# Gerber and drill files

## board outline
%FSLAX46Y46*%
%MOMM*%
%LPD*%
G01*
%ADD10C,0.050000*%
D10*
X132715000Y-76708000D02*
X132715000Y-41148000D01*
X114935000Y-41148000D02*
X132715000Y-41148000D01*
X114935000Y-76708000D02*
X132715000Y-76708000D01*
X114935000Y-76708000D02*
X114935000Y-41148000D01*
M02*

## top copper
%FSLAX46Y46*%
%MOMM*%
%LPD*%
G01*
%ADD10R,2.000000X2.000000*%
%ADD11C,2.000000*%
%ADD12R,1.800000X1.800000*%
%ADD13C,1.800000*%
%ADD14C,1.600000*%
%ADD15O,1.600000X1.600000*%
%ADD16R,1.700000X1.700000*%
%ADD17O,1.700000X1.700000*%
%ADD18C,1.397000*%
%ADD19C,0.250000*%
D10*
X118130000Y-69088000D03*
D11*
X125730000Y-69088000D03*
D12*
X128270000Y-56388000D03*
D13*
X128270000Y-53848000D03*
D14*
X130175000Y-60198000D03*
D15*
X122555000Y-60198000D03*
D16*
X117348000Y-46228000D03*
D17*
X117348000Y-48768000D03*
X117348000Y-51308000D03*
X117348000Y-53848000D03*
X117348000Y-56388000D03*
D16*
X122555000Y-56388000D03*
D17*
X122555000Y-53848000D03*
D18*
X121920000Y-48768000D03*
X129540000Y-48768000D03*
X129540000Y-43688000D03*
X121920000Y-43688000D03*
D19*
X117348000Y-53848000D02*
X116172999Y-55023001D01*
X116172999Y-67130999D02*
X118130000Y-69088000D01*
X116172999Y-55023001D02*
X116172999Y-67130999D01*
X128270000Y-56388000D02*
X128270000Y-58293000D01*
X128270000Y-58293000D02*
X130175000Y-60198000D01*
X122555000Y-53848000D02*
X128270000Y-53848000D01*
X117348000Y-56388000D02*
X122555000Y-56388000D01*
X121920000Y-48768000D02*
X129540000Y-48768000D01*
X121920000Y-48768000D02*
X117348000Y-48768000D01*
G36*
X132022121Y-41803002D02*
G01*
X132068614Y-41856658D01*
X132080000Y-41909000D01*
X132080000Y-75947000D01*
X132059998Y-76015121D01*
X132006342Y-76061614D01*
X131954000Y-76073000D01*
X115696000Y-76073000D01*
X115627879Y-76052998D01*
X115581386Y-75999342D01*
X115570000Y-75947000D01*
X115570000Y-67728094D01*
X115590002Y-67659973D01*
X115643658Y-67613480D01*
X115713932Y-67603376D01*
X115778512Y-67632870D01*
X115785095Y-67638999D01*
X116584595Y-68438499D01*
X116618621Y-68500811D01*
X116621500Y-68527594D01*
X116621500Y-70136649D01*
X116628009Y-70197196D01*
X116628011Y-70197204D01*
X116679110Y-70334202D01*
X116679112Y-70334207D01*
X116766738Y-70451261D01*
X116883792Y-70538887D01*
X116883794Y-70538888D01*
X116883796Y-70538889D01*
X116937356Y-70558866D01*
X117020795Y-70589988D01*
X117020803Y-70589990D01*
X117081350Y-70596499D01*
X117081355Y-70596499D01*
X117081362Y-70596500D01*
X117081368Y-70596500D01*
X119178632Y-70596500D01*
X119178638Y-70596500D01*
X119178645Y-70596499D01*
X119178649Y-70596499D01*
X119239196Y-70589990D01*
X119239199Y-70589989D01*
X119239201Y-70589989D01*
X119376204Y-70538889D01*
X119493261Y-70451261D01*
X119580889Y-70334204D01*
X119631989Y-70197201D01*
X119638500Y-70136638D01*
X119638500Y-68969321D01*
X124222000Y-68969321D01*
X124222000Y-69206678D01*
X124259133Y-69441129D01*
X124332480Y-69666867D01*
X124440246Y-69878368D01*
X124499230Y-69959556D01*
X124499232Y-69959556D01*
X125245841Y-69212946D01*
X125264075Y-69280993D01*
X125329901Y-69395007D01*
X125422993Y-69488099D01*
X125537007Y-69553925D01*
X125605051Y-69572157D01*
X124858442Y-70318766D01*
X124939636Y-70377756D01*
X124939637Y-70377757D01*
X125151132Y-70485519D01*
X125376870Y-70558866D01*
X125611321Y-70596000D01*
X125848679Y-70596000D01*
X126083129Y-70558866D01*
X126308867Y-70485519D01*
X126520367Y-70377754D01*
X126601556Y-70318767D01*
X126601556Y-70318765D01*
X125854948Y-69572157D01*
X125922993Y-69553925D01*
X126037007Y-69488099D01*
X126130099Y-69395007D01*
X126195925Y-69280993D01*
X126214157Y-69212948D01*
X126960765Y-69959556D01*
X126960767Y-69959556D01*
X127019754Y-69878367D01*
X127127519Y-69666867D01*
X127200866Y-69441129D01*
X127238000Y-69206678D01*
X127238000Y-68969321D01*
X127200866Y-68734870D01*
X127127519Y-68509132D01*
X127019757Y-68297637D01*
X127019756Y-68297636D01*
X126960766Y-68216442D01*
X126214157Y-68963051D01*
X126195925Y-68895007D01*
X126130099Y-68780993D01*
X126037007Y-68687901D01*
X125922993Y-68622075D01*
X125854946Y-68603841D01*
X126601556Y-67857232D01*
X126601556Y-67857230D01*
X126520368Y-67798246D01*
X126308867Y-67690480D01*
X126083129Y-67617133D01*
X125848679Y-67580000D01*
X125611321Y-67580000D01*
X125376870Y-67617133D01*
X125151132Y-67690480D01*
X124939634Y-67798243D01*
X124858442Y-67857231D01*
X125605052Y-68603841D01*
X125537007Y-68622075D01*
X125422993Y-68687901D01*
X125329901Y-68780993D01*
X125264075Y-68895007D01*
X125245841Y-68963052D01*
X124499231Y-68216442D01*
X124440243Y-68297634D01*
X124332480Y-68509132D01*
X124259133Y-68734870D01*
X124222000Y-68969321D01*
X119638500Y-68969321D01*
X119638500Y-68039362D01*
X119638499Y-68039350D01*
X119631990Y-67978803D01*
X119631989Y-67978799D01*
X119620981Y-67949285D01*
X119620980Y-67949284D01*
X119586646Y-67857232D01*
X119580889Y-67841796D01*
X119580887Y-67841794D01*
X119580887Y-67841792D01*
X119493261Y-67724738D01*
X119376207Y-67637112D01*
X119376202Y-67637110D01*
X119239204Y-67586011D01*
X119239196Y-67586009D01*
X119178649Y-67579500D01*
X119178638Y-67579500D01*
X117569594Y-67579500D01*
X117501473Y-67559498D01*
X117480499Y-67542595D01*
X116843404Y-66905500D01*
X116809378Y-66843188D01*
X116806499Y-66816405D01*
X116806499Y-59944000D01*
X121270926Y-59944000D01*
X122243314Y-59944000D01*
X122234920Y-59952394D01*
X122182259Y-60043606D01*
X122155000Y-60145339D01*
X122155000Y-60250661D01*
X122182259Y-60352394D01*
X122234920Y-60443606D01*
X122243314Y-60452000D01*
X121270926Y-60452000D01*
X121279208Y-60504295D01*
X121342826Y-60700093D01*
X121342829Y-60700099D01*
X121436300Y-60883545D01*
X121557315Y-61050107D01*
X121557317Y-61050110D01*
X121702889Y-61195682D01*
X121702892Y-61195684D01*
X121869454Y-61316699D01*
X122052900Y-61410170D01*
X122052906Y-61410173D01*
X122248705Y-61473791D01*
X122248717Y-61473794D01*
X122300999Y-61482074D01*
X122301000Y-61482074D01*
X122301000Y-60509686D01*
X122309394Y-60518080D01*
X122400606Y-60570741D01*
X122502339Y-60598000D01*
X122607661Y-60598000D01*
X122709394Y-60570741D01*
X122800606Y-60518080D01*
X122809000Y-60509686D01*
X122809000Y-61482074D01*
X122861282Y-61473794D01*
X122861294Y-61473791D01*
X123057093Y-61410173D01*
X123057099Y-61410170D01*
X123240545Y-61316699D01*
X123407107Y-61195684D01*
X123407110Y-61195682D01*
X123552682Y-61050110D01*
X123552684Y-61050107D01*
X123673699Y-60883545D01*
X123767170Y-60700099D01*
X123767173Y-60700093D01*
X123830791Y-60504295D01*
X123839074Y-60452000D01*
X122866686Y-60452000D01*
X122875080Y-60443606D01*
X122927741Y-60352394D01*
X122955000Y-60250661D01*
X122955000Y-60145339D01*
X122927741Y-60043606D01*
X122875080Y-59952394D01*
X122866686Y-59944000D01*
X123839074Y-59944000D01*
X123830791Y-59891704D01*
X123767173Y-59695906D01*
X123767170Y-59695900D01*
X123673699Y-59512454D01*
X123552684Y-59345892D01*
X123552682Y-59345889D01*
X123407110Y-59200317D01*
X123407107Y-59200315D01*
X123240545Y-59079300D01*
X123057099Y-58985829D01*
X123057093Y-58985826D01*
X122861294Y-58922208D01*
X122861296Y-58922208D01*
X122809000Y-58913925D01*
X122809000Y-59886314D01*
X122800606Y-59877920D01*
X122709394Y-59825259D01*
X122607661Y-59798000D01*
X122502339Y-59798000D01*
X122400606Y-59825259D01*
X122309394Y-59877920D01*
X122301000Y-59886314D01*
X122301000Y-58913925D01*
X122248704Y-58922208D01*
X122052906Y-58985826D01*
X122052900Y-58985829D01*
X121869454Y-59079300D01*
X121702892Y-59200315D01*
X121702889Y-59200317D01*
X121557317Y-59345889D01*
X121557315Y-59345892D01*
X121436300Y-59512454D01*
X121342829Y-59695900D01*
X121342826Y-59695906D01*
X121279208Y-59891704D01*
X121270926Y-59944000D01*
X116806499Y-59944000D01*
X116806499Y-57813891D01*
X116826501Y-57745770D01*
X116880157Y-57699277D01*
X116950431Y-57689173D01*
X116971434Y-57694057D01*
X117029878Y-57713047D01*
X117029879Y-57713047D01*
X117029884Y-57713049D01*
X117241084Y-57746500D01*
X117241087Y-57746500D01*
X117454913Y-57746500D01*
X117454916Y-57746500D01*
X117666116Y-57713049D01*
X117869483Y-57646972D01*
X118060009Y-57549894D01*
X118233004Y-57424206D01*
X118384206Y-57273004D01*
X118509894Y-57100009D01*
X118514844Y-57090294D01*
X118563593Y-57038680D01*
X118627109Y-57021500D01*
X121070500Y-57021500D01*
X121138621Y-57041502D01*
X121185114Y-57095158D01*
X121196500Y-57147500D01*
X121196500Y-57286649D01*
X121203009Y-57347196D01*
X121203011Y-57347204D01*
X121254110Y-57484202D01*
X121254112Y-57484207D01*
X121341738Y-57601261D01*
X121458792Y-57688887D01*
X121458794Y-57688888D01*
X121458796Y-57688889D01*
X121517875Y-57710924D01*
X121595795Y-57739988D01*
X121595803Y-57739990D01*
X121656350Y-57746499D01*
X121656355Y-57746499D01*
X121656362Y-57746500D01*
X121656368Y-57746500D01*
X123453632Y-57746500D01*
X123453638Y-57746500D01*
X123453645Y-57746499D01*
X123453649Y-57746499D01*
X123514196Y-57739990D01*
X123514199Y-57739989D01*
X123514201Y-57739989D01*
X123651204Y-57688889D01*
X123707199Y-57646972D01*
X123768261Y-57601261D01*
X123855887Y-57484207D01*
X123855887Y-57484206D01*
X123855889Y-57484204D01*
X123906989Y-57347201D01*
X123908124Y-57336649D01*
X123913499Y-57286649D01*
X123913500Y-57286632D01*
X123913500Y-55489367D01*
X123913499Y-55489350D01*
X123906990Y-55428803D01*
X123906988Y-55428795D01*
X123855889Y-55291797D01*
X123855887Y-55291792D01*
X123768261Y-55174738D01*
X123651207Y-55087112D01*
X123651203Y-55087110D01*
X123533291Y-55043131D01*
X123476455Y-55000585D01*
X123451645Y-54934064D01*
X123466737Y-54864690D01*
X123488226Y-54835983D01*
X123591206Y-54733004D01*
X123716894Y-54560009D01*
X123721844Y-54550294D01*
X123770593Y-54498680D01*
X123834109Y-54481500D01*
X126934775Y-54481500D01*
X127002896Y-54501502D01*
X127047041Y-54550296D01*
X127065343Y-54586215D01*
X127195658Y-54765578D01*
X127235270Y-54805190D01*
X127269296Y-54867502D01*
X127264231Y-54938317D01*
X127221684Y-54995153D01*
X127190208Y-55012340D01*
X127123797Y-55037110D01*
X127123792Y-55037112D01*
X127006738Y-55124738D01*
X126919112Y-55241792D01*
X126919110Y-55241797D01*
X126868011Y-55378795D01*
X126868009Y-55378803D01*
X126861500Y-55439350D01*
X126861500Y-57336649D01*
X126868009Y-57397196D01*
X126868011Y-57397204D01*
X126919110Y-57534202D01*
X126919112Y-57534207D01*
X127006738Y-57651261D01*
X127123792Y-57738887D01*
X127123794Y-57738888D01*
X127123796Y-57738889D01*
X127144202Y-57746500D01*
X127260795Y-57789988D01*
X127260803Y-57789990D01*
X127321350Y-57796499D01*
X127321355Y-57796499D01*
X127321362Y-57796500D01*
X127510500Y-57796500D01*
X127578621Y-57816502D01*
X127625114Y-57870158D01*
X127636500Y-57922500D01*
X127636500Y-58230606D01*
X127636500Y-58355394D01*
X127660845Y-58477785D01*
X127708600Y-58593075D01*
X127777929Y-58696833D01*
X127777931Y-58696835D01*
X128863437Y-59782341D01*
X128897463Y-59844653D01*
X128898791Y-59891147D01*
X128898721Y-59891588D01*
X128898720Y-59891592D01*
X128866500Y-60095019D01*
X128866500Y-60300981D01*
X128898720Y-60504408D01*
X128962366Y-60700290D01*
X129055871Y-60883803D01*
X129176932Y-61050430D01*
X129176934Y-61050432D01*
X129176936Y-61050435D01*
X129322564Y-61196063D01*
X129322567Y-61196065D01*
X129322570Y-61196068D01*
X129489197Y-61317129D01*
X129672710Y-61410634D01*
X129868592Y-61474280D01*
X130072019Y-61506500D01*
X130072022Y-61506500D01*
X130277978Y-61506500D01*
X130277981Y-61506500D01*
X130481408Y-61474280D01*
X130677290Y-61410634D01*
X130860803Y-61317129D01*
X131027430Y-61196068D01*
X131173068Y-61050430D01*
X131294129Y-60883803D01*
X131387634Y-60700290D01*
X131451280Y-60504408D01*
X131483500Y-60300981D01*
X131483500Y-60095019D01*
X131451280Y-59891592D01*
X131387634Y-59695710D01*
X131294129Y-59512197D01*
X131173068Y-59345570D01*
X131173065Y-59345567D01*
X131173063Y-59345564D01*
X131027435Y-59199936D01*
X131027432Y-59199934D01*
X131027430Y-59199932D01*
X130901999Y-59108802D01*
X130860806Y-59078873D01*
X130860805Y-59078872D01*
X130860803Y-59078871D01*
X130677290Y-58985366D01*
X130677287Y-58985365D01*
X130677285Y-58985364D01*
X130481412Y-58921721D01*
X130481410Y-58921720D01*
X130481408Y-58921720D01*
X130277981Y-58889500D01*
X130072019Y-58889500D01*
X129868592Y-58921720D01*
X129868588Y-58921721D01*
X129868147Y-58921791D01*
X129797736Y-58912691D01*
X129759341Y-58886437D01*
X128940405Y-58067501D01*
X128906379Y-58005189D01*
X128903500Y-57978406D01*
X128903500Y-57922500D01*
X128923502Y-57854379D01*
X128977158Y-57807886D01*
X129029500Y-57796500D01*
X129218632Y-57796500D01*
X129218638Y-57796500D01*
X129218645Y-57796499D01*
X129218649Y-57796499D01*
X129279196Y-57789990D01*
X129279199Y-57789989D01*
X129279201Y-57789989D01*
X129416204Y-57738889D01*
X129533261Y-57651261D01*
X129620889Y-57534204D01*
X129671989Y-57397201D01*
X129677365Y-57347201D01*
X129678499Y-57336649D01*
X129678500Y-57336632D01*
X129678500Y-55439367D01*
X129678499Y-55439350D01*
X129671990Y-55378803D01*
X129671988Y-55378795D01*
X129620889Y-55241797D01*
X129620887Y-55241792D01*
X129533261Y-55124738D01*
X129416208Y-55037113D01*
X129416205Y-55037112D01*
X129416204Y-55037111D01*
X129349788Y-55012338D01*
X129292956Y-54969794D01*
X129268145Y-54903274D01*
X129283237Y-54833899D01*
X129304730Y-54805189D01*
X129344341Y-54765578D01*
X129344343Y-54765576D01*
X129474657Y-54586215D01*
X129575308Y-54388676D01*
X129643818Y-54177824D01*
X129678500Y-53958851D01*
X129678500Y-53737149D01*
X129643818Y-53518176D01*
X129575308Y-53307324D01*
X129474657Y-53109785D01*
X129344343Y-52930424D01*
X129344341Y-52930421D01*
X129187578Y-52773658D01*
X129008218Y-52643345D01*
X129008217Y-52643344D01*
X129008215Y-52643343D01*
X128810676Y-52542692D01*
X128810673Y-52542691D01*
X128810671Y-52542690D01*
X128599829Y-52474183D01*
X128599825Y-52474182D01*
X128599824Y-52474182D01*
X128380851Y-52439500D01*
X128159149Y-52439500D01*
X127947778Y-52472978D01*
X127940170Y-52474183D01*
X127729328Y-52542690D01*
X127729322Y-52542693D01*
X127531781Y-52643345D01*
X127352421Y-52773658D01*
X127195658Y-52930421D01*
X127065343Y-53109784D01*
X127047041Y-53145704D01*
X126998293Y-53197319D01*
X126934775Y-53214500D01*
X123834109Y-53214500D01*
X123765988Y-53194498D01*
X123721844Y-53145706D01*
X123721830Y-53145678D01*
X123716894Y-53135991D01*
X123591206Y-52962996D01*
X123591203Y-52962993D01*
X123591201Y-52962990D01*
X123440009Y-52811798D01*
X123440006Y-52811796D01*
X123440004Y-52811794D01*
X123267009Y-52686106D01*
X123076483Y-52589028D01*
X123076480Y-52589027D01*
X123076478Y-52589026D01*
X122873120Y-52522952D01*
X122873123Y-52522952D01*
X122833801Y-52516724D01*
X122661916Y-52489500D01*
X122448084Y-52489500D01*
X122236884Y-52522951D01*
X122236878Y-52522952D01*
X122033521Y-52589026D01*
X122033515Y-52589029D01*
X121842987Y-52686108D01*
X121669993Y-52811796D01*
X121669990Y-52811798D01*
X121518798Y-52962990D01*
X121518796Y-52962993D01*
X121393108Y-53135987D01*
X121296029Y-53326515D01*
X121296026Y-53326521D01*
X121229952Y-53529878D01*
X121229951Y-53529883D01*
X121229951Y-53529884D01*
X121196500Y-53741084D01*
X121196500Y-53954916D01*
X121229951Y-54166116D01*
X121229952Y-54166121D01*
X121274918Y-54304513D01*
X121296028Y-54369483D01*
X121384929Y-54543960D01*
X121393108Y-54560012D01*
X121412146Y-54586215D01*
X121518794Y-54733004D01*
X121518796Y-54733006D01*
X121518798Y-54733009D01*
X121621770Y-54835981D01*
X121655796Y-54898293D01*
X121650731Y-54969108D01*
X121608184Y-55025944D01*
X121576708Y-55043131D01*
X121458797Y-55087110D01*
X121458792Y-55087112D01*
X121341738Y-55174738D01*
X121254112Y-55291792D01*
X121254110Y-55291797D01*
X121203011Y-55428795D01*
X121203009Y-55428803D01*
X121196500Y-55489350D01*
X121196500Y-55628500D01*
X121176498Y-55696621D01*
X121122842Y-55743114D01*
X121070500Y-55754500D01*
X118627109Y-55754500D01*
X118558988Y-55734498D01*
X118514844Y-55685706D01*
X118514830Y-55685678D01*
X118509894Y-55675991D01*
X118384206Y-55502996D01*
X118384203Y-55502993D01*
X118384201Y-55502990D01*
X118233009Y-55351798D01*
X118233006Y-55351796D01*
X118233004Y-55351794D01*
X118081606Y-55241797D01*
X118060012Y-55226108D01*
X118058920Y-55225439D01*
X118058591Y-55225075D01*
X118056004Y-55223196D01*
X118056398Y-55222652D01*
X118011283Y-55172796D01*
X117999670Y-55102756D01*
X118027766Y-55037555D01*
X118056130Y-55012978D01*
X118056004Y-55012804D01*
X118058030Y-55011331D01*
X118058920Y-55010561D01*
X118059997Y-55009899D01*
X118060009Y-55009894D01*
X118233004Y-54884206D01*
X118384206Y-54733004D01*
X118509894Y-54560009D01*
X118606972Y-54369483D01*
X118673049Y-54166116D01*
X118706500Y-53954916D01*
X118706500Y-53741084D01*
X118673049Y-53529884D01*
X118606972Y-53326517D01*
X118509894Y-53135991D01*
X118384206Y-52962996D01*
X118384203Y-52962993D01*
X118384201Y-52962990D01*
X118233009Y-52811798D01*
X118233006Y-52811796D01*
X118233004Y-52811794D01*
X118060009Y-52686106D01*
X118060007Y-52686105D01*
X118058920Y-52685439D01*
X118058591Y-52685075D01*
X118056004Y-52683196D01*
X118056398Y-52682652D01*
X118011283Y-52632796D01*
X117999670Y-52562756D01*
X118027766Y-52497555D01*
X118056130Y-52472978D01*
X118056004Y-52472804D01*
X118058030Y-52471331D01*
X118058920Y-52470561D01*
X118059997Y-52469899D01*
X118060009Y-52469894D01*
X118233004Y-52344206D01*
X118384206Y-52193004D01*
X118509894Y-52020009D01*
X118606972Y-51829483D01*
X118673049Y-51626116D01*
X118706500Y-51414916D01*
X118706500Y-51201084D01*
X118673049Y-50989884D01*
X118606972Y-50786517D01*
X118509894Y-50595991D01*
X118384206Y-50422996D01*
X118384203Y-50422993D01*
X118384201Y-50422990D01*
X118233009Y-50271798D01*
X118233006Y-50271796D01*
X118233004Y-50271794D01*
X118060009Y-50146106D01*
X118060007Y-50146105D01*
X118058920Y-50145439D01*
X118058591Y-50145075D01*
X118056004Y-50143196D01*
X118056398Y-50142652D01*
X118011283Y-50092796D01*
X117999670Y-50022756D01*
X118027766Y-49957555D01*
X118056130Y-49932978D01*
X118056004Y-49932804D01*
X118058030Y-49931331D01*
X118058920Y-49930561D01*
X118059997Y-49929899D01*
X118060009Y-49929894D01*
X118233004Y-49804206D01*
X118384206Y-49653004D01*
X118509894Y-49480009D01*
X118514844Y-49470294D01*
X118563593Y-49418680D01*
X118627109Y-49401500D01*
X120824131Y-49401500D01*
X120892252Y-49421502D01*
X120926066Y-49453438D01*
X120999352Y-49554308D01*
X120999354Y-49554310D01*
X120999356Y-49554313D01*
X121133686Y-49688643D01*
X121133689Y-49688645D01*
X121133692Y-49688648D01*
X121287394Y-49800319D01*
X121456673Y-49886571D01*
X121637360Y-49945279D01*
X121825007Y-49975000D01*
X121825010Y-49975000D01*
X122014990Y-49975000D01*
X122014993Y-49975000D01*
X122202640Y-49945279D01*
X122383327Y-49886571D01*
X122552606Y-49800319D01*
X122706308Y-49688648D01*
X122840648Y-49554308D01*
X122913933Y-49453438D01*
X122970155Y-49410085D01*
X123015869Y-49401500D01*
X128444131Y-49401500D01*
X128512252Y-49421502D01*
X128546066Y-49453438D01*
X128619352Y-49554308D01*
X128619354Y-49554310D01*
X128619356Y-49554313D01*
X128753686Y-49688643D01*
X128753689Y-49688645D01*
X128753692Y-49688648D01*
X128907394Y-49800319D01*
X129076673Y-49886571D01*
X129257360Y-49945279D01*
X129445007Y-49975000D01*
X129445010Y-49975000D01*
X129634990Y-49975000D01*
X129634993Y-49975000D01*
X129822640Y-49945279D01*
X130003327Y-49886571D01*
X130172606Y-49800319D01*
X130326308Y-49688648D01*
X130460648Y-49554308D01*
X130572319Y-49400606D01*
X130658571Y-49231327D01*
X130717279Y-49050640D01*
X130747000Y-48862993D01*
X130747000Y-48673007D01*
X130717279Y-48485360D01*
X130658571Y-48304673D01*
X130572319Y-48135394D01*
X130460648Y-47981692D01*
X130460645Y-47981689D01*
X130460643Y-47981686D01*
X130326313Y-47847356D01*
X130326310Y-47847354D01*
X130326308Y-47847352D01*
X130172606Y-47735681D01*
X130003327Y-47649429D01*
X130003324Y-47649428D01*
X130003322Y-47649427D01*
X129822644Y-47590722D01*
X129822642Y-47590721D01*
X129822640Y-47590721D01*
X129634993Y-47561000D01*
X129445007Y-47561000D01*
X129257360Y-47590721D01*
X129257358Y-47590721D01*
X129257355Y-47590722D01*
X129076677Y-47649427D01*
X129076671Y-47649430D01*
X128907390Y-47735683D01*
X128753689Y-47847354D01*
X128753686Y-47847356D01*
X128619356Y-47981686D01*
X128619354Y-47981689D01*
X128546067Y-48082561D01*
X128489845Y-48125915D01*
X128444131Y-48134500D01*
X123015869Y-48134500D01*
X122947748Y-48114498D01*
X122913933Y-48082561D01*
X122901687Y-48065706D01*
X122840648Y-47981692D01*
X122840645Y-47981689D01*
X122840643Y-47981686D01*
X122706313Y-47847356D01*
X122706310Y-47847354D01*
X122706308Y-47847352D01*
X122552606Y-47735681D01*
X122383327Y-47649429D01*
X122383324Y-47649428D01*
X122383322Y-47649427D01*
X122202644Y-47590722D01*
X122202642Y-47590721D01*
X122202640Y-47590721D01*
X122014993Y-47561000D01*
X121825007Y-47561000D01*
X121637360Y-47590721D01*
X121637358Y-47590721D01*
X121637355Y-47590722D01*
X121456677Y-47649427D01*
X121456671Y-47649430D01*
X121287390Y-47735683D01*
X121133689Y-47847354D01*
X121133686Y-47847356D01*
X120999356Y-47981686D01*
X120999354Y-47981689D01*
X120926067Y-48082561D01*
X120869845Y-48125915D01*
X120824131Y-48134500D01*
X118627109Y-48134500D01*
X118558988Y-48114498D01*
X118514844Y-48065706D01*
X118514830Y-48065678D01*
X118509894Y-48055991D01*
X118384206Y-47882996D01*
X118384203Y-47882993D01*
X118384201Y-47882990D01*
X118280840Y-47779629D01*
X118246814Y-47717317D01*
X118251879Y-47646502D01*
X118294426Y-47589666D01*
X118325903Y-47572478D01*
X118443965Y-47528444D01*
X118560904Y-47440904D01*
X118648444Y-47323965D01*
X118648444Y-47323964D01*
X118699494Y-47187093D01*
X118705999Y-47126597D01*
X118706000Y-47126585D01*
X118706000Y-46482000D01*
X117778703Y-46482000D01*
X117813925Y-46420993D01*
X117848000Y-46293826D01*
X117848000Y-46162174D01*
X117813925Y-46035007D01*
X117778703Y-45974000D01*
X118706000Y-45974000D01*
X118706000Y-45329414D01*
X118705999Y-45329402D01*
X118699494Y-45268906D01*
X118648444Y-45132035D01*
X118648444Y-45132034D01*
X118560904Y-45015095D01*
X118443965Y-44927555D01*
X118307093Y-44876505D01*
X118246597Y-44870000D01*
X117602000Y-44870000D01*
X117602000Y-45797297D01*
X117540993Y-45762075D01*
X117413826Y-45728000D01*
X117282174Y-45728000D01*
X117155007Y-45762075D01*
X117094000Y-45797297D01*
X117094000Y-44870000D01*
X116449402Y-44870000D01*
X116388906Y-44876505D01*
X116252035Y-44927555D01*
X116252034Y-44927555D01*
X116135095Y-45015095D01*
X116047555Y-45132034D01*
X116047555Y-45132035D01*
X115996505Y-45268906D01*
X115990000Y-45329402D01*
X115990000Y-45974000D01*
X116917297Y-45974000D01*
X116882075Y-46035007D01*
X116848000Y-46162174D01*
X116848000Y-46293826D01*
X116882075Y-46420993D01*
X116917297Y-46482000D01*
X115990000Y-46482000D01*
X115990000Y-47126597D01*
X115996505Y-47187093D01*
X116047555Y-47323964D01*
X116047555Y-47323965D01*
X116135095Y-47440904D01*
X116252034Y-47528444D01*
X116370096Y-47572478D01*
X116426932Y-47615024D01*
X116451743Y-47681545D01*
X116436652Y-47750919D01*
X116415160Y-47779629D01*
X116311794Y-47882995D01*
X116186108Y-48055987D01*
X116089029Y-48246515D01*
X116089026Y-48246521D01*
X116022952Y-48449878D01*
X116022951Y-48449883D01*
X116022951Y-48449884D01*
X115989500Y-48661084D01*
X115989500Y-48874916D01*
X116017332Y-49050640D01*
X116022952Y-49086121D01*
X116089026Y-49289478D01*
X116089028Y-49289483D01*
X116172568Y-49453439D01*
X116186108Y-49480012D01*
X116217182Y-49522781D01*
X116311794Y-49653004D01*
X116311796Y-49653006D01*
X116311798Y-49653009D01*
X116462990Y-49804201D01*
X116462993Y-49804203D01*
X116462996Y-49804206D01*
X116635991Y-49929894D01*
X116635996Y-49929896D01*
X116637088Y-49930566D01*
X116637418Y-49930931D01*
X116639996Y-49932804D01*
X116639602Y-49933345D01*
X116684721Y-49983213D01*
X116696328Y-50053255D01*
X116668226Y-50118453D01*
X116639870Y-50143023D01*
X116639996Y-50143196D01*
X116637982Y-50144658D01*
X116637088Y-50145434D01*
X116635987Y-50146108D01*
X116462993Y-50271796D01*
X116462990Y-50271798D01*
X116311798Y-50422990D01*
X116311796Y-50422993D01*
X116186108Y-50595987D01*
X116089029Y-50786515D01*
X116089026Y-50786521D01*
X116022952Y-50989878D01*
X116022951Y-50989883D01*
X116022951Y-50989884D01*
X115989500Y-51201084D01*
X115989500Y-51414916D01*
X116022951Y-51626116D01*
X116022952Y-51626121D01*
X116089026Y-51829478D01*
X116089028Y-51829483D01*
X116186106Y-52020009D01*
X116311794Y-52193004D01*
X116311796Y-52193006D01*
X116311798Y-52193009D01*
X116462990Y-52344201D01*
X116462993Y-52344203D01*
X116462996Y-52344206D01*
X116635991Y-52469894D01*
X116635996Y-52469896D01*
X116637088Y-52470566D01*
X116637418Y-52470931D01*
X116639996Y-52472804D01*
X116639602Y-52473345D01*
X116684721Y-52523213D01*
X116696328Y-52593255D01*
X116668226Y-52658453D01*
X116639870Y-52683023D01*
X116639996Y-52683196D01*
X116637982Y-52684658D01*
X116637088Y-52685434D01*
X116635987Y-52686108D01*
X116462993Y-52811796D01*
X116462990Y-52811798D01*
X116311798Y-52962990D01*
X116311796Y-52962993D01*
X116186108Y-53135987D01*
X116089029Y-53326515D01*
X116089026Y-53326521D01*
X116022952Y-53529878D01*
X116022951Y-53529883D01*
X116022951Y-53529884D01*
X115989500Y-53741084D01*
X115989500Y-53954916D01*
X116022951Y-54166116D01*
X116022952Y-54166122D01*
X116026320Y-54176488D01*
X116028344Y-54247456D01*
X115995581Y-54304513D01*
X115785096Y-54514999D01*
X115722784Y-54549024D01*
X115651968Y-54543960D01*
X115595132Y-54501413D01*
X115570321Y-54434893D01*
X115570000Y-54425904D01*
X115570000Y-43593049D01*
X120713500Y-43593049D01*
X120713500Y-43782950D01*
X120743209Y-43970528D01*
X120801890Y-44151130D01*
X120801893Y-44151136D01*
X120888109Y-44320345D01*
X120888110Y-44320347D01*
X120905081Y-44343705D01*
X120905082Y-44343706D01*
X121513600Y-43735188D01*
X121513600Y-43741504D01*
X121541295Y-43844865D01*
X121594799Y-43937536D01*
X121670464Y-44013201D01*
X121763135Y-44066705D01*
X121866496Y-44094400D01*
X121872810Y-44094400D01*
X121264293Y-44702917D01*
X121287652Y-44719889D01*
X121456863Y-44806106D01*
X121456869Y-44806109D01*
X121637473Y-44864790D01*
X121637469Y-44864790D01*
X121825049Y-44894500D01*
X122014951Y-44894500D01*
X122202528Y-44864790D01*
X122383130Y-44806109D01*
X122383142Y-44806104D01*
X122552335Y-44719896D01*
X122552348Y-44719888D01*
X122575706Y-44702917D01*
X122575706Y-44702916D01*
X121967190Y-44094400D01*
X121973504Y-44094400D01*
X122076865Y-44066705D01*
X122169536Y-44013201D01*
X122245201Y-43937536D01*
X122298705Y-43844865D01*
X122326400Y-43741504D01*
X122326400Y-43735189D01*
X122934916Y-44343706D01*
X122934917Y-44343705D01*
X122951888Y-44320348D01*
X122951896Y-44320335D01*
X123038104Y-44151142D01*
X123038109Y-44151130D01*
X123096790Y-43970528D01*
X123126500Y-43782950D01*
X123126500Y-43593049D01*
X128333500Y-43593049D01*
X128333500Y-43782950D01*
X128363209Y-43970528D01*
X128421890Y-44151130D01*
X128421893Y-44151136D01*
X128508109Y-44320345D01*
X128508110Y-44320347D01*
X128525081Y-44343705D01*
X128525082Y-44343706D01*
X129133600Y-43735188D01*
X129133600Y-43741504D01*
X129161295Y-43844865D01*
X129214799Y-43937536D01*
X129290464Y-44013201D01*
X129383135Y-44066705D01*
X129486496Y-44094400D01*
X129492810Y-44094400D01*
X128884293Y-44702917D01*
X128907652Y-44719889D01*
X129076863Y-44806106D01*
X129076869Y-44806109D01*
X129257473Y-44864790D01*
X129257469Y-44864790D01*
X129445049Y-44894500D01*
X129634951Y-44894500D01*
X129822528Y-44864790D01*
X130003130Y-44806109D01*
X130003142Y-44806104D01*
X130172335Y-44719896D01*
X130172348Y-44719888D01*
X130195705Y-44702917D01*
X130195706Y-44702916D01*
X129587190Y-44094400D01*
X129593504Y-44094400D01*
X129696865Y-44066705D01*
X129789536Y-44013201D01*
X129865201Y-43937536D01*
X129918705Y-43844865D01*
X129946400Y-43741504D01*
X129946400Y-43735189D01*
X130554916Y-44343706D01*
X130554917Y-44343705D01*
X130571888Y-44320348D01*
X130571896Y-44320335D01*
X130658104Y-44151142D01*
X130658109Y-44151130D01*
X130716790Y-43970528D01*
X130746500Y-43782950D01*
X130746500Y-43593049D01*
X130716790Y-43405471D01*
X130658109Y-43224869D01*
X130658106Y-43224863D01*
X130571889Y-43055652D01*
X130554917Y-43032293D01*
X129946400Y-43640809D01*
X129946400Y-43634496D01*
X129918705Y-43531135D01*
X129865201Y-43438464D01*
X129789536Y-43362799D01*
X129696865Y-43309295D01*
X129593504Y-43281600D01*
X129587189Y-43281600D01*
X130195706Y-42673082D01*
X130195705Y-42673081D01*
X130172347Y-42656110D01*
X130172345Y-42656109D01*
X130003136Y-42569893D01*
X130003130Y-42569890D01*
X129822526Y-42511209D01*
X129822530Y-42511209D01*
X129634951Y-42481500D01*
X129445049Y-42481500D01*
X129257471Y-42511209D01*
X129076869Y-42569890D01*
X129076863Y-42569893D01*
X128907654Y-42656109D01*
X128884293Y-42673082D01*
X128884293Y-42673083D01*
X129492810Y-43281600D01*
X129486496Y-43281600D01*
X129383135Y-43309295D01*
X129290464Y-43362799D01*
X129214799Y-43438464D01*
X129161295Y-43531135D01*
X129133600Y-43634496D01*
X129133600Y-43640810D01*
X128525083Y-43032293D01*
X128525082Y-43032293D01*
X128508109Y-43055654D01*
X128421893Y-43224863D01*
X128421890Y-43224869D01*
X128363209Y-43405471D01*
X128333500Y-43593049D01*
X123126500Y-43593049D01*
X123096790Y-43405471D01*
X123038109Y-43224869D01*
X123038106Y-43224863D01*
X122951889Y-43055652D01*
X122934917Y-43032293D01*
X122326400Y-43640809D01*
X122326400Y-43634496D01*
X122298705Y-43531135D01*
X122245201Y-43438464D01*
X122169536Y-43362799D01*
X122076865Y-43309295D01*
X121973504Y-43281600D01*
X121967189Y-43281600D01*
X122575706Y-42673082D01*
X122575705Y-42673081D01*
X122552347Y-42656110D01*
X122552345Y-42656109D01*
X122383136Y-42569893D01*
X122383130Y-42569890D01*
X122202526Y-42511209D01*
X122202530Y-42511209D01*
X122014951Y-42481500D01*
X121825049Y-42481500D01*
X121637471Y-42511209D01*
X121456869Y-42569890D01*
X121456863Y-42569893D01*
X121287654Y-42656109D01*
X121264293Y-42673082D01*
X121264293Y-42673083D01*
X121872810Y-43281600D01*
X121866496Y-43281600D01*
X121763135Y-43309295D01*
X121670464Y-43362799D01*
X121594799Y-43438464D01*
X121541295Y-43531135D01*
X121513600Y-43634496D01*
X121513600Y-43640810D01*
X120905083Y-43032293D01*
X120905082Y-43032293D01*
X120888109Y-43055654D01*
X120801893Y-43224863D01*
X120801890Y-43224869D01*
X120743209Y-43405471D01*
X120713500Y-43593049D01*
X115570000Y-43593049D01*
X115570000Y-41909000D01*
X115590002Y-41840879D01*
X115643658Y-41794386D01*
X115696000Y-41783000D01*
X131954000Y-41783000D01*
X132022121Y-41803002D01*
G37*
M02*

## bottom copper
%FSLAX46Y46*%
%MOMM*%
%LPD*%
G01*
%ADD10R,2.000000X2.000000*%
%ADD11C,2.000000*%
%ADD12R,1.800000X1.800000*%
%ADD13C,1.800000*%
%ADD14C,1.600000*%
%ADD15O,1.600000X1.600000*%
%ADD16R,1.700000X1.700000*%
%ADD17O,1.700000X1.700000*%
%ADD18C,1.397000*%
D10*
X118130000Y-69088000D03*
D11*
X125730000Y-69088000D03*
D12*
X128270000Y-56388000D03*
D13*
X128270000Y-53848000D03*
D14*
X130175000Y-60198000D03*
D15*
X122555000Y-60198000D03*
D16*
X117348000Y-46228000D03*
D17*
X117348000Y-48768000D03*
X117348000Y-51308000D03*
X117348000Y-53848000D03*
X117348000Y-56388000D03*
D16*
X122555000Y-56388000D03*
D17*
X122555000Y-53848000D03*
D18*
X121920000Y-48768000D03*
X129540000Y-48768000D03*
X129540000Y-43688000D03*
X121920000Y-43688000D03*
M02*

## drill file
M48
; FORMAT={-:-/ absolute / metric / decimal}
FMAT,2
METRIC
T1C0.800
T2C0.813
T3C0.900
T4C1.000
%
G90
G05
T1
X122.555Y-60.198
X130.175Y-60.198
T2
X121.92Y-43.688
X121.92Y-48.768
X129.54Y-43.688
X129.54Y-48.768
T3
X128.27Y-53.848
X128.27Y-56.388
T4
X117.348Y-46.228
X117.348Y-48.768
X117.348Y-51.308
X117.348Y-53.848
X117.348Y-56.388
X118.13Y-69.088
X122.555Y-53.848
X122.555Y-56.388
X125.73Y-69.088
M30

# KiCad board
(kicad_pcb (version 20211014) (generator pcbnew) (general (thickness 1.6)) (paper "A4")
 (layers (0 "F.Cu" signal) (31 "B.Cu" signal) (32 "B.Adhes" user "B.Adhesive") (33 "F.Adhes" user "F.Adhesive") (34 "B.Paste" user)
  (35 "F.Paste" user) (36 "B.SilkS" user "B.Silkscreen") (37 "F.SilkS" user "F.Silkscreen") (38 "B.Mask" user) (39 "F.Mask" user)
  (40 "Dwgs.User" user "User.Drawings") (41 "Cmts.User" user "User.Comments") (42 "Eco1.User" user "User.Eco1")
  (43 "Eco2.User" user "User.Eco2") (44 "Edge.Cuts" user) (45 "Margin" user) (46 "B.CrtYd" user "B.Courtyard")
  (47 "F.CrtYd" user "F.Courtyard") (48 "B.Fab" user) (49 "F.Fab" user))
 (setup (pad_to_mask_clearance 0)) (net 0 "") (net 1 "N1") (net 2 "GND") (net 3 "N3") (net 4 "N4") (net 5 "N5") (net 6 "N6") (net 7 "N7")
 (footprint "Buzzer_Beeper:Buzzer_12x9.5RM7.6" (layer "F.Cu") (at 118.13 69.088)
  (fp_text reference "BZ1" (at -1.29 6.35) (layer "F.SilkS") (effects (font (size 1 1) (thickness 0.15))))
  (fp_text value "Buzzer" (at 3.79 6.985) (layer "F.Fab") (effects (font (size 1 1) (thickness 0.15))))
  (pad "1" thru_hole rect locked (at 0 0) (size 2 2) (drill 1) (layers *.Cu *.Mask) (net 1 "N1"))
  (pad "2" thru_hole circle locked (at 7.6 0) (size 2 2) (drill 1) (layers *.Cu *.Mask) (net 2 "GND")))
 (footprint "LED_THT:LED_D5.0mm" (layer "F.Cu") (at 128.27 56.388 90)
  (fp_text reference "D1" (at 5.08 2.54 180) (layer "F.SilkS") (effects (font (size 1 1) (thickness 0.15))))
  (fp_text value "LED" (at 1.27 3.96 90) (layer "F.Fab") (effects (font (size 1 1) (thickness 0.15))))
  (pad "1" thru_hole rect locked (at 0 0 90) (size 1.8 1.8) (drill 0.9) (layers *.Cu *.Mask) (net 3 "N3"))
  (pad "2" thru_hole circle locked (at 2.54 0 90) (size 1.8 1.8) (drill 0.9) (layers *.Cu *.Mask) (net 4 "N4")))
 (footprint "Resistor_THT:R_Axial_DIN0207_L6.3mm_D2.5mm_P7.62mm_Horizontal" (layer "F.Cu") (at 130.175 60.198 180)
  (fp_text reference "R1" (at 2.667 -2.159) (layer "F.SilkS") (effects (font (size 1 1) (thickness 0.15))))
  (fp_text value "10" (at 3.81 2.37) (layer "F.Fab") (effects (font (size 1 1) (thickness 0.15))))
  (pad "1" thru_hole circle locked (at 0 0 180) (size 1.6 1.6) (drill 0.8) (layers *.Cu *.Mask) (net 3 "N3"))
  (pad "2" thru_hole oval locked (at 7.62 0 180) (size 1.6 1.6) (drill 0.8) (layers *.Cu *.Mask) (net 2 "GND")))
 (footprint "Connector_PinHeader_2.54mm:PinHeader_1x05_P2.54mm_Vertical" (layer "F.Cu") (at 117.348 46.228)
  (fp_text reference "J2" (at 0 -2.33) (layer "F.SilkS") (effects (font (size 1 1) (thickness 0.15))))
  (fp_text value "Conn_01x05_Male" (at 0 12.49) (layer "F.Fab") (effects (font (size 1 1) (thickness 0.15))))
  (pad "1" thru_hole rect locked (at 0 0) (size 1.7 1.7) (drill 1) (layers *.Cu *.Mask) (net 2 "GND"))
  (pad "2" thru_hole oval locked (at 0 2.54) (size 1.7 1.7) (drill 1) (layers *.Cu *.Mask) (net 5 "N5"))
  (pad "3" thru_hole oval locked (at 0 5.08) (size 1.7 1.7) (drill 1) (layers *.Cu *.Mask) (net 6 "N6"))
  (pad "4" thru_hole oval locked (at 0 7.62) (size 1.7 1.7) (drill 1) (layers *.Cu *.Mask) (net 1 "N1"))
  (pad "5" thru_hole oval locked (at 0 10.16) (size 1.7 1.7) (drill 1) (layers *.Cu *.Mask) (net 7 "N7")))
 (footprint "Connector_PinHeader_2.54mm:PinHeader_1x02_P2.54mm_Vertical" (layer "F.Cu") (at 122.555 56.388 180)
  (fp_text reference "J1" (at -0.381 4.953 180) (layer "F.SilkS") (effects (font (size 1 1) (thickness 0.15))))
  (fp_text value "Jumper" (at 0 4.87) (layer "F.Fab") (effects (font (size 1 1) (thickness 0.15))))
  (pad "1" thru_hole rect locked (at 0 0 180) (size 1.7 1.7) (drill 1) (layers *.Cu *.Mask) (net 7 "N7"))
  (pad "2" thru_hole oval locked (at 0 2.54 180) (size 1.7 1.7) (drill 1) (layers *.Cu *.Mask) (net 4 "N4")))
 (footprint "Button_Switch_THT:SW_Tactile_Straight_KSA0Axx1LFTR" (layer "F.Cu") (at 129.54 48.768 180)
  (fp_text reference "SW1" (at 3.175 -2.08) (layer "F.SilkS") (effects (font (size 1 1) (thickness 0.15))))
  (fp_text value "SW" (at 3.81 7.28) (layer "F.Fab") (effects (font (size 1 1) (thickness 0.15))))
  (pad "1" thru_hole circle locked (at 7.62 0 180) (size 1.397 1.397) (drill 0.8128) (layers *.Cu *.Mask) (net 5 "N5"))
  (pad "1" thru_hole circle locked (at 0 0 180) (size 1.397 1.397) (drill 0.8128) (layers *.Cu *.Mask) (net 5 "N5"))
  (pad "2" thru_hole circle locked (at 0 5.08 180) (size 1.397 1.397) (drill 0.8128) (layers *.Cu *.Mask) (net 2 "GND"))
  (pad "2" thru_hole circle locked (at 7.62 5.08 180) (size 1.397 1.397) (drill 0.8128) (layers *.Cu *.Mask) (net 2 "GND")))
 (gr_line (start 132.715 76.708) (end 132.715 41.148) (layer "Edge.Cuts") (width 0.05))
 (gr_line (start 114.935 41.148) (end 132.715 41.148) (layer "Edge.Cuts") (width 0.05))
 (gr_line (start 114.935 76.708) (end 132.715 76.708) (layer "Edge.Cuts") (width 0.05))
 (gr_line (start 114.935 76.708) (end 114.935 41.148) (layer "Edge.Cuts") (width 0.05))
 (segment (start 117.348 53.848) (end 116.172999 55.023001) (width 0.25) (layer "F.Cu") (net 1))
 (segment (start 116.172999 67.130999) (end 118.13 69.088) (width 0.25) (layer "F.Cu") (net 1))
 (segment (start 116.172999 55.023001) (end 116.172999 67.130999) (width 0.25) (layer "F.Cu") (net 1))
 (segment (start 128.27 56.388) (end 128.27 58.293) (width 0.25) (layer "F.Cu") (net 3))
 (segment (start 128.27 58.293) (end 130.175 60.198) (width 0.25) (layer "F.Cu") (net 3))
 (segment (start 122.555 53.848) (end 128.27 53.848) (width 0.25) (layer "F.Cu") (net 4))
 (segment (start 117.348 56.388) (end 122.555 56.388) (width 0.25) (layer "F.Cu") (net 7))
 (segment (start 121.92 48.768) (end 129.54 48.768) (width 0.25) (layer "F.Cu") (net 5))
 (segment (start 121.92 48.768) (end 117.348 48.768) (width 0.25) (layer "F.Cu") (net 5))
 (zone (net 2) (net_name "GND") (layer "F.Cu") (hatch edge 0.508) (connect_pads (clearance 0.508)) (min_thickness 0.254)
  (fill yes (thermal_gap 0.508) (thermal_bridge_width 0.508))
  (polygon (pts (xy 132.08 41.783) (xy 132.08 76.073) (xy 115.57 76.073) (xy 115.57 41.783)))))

